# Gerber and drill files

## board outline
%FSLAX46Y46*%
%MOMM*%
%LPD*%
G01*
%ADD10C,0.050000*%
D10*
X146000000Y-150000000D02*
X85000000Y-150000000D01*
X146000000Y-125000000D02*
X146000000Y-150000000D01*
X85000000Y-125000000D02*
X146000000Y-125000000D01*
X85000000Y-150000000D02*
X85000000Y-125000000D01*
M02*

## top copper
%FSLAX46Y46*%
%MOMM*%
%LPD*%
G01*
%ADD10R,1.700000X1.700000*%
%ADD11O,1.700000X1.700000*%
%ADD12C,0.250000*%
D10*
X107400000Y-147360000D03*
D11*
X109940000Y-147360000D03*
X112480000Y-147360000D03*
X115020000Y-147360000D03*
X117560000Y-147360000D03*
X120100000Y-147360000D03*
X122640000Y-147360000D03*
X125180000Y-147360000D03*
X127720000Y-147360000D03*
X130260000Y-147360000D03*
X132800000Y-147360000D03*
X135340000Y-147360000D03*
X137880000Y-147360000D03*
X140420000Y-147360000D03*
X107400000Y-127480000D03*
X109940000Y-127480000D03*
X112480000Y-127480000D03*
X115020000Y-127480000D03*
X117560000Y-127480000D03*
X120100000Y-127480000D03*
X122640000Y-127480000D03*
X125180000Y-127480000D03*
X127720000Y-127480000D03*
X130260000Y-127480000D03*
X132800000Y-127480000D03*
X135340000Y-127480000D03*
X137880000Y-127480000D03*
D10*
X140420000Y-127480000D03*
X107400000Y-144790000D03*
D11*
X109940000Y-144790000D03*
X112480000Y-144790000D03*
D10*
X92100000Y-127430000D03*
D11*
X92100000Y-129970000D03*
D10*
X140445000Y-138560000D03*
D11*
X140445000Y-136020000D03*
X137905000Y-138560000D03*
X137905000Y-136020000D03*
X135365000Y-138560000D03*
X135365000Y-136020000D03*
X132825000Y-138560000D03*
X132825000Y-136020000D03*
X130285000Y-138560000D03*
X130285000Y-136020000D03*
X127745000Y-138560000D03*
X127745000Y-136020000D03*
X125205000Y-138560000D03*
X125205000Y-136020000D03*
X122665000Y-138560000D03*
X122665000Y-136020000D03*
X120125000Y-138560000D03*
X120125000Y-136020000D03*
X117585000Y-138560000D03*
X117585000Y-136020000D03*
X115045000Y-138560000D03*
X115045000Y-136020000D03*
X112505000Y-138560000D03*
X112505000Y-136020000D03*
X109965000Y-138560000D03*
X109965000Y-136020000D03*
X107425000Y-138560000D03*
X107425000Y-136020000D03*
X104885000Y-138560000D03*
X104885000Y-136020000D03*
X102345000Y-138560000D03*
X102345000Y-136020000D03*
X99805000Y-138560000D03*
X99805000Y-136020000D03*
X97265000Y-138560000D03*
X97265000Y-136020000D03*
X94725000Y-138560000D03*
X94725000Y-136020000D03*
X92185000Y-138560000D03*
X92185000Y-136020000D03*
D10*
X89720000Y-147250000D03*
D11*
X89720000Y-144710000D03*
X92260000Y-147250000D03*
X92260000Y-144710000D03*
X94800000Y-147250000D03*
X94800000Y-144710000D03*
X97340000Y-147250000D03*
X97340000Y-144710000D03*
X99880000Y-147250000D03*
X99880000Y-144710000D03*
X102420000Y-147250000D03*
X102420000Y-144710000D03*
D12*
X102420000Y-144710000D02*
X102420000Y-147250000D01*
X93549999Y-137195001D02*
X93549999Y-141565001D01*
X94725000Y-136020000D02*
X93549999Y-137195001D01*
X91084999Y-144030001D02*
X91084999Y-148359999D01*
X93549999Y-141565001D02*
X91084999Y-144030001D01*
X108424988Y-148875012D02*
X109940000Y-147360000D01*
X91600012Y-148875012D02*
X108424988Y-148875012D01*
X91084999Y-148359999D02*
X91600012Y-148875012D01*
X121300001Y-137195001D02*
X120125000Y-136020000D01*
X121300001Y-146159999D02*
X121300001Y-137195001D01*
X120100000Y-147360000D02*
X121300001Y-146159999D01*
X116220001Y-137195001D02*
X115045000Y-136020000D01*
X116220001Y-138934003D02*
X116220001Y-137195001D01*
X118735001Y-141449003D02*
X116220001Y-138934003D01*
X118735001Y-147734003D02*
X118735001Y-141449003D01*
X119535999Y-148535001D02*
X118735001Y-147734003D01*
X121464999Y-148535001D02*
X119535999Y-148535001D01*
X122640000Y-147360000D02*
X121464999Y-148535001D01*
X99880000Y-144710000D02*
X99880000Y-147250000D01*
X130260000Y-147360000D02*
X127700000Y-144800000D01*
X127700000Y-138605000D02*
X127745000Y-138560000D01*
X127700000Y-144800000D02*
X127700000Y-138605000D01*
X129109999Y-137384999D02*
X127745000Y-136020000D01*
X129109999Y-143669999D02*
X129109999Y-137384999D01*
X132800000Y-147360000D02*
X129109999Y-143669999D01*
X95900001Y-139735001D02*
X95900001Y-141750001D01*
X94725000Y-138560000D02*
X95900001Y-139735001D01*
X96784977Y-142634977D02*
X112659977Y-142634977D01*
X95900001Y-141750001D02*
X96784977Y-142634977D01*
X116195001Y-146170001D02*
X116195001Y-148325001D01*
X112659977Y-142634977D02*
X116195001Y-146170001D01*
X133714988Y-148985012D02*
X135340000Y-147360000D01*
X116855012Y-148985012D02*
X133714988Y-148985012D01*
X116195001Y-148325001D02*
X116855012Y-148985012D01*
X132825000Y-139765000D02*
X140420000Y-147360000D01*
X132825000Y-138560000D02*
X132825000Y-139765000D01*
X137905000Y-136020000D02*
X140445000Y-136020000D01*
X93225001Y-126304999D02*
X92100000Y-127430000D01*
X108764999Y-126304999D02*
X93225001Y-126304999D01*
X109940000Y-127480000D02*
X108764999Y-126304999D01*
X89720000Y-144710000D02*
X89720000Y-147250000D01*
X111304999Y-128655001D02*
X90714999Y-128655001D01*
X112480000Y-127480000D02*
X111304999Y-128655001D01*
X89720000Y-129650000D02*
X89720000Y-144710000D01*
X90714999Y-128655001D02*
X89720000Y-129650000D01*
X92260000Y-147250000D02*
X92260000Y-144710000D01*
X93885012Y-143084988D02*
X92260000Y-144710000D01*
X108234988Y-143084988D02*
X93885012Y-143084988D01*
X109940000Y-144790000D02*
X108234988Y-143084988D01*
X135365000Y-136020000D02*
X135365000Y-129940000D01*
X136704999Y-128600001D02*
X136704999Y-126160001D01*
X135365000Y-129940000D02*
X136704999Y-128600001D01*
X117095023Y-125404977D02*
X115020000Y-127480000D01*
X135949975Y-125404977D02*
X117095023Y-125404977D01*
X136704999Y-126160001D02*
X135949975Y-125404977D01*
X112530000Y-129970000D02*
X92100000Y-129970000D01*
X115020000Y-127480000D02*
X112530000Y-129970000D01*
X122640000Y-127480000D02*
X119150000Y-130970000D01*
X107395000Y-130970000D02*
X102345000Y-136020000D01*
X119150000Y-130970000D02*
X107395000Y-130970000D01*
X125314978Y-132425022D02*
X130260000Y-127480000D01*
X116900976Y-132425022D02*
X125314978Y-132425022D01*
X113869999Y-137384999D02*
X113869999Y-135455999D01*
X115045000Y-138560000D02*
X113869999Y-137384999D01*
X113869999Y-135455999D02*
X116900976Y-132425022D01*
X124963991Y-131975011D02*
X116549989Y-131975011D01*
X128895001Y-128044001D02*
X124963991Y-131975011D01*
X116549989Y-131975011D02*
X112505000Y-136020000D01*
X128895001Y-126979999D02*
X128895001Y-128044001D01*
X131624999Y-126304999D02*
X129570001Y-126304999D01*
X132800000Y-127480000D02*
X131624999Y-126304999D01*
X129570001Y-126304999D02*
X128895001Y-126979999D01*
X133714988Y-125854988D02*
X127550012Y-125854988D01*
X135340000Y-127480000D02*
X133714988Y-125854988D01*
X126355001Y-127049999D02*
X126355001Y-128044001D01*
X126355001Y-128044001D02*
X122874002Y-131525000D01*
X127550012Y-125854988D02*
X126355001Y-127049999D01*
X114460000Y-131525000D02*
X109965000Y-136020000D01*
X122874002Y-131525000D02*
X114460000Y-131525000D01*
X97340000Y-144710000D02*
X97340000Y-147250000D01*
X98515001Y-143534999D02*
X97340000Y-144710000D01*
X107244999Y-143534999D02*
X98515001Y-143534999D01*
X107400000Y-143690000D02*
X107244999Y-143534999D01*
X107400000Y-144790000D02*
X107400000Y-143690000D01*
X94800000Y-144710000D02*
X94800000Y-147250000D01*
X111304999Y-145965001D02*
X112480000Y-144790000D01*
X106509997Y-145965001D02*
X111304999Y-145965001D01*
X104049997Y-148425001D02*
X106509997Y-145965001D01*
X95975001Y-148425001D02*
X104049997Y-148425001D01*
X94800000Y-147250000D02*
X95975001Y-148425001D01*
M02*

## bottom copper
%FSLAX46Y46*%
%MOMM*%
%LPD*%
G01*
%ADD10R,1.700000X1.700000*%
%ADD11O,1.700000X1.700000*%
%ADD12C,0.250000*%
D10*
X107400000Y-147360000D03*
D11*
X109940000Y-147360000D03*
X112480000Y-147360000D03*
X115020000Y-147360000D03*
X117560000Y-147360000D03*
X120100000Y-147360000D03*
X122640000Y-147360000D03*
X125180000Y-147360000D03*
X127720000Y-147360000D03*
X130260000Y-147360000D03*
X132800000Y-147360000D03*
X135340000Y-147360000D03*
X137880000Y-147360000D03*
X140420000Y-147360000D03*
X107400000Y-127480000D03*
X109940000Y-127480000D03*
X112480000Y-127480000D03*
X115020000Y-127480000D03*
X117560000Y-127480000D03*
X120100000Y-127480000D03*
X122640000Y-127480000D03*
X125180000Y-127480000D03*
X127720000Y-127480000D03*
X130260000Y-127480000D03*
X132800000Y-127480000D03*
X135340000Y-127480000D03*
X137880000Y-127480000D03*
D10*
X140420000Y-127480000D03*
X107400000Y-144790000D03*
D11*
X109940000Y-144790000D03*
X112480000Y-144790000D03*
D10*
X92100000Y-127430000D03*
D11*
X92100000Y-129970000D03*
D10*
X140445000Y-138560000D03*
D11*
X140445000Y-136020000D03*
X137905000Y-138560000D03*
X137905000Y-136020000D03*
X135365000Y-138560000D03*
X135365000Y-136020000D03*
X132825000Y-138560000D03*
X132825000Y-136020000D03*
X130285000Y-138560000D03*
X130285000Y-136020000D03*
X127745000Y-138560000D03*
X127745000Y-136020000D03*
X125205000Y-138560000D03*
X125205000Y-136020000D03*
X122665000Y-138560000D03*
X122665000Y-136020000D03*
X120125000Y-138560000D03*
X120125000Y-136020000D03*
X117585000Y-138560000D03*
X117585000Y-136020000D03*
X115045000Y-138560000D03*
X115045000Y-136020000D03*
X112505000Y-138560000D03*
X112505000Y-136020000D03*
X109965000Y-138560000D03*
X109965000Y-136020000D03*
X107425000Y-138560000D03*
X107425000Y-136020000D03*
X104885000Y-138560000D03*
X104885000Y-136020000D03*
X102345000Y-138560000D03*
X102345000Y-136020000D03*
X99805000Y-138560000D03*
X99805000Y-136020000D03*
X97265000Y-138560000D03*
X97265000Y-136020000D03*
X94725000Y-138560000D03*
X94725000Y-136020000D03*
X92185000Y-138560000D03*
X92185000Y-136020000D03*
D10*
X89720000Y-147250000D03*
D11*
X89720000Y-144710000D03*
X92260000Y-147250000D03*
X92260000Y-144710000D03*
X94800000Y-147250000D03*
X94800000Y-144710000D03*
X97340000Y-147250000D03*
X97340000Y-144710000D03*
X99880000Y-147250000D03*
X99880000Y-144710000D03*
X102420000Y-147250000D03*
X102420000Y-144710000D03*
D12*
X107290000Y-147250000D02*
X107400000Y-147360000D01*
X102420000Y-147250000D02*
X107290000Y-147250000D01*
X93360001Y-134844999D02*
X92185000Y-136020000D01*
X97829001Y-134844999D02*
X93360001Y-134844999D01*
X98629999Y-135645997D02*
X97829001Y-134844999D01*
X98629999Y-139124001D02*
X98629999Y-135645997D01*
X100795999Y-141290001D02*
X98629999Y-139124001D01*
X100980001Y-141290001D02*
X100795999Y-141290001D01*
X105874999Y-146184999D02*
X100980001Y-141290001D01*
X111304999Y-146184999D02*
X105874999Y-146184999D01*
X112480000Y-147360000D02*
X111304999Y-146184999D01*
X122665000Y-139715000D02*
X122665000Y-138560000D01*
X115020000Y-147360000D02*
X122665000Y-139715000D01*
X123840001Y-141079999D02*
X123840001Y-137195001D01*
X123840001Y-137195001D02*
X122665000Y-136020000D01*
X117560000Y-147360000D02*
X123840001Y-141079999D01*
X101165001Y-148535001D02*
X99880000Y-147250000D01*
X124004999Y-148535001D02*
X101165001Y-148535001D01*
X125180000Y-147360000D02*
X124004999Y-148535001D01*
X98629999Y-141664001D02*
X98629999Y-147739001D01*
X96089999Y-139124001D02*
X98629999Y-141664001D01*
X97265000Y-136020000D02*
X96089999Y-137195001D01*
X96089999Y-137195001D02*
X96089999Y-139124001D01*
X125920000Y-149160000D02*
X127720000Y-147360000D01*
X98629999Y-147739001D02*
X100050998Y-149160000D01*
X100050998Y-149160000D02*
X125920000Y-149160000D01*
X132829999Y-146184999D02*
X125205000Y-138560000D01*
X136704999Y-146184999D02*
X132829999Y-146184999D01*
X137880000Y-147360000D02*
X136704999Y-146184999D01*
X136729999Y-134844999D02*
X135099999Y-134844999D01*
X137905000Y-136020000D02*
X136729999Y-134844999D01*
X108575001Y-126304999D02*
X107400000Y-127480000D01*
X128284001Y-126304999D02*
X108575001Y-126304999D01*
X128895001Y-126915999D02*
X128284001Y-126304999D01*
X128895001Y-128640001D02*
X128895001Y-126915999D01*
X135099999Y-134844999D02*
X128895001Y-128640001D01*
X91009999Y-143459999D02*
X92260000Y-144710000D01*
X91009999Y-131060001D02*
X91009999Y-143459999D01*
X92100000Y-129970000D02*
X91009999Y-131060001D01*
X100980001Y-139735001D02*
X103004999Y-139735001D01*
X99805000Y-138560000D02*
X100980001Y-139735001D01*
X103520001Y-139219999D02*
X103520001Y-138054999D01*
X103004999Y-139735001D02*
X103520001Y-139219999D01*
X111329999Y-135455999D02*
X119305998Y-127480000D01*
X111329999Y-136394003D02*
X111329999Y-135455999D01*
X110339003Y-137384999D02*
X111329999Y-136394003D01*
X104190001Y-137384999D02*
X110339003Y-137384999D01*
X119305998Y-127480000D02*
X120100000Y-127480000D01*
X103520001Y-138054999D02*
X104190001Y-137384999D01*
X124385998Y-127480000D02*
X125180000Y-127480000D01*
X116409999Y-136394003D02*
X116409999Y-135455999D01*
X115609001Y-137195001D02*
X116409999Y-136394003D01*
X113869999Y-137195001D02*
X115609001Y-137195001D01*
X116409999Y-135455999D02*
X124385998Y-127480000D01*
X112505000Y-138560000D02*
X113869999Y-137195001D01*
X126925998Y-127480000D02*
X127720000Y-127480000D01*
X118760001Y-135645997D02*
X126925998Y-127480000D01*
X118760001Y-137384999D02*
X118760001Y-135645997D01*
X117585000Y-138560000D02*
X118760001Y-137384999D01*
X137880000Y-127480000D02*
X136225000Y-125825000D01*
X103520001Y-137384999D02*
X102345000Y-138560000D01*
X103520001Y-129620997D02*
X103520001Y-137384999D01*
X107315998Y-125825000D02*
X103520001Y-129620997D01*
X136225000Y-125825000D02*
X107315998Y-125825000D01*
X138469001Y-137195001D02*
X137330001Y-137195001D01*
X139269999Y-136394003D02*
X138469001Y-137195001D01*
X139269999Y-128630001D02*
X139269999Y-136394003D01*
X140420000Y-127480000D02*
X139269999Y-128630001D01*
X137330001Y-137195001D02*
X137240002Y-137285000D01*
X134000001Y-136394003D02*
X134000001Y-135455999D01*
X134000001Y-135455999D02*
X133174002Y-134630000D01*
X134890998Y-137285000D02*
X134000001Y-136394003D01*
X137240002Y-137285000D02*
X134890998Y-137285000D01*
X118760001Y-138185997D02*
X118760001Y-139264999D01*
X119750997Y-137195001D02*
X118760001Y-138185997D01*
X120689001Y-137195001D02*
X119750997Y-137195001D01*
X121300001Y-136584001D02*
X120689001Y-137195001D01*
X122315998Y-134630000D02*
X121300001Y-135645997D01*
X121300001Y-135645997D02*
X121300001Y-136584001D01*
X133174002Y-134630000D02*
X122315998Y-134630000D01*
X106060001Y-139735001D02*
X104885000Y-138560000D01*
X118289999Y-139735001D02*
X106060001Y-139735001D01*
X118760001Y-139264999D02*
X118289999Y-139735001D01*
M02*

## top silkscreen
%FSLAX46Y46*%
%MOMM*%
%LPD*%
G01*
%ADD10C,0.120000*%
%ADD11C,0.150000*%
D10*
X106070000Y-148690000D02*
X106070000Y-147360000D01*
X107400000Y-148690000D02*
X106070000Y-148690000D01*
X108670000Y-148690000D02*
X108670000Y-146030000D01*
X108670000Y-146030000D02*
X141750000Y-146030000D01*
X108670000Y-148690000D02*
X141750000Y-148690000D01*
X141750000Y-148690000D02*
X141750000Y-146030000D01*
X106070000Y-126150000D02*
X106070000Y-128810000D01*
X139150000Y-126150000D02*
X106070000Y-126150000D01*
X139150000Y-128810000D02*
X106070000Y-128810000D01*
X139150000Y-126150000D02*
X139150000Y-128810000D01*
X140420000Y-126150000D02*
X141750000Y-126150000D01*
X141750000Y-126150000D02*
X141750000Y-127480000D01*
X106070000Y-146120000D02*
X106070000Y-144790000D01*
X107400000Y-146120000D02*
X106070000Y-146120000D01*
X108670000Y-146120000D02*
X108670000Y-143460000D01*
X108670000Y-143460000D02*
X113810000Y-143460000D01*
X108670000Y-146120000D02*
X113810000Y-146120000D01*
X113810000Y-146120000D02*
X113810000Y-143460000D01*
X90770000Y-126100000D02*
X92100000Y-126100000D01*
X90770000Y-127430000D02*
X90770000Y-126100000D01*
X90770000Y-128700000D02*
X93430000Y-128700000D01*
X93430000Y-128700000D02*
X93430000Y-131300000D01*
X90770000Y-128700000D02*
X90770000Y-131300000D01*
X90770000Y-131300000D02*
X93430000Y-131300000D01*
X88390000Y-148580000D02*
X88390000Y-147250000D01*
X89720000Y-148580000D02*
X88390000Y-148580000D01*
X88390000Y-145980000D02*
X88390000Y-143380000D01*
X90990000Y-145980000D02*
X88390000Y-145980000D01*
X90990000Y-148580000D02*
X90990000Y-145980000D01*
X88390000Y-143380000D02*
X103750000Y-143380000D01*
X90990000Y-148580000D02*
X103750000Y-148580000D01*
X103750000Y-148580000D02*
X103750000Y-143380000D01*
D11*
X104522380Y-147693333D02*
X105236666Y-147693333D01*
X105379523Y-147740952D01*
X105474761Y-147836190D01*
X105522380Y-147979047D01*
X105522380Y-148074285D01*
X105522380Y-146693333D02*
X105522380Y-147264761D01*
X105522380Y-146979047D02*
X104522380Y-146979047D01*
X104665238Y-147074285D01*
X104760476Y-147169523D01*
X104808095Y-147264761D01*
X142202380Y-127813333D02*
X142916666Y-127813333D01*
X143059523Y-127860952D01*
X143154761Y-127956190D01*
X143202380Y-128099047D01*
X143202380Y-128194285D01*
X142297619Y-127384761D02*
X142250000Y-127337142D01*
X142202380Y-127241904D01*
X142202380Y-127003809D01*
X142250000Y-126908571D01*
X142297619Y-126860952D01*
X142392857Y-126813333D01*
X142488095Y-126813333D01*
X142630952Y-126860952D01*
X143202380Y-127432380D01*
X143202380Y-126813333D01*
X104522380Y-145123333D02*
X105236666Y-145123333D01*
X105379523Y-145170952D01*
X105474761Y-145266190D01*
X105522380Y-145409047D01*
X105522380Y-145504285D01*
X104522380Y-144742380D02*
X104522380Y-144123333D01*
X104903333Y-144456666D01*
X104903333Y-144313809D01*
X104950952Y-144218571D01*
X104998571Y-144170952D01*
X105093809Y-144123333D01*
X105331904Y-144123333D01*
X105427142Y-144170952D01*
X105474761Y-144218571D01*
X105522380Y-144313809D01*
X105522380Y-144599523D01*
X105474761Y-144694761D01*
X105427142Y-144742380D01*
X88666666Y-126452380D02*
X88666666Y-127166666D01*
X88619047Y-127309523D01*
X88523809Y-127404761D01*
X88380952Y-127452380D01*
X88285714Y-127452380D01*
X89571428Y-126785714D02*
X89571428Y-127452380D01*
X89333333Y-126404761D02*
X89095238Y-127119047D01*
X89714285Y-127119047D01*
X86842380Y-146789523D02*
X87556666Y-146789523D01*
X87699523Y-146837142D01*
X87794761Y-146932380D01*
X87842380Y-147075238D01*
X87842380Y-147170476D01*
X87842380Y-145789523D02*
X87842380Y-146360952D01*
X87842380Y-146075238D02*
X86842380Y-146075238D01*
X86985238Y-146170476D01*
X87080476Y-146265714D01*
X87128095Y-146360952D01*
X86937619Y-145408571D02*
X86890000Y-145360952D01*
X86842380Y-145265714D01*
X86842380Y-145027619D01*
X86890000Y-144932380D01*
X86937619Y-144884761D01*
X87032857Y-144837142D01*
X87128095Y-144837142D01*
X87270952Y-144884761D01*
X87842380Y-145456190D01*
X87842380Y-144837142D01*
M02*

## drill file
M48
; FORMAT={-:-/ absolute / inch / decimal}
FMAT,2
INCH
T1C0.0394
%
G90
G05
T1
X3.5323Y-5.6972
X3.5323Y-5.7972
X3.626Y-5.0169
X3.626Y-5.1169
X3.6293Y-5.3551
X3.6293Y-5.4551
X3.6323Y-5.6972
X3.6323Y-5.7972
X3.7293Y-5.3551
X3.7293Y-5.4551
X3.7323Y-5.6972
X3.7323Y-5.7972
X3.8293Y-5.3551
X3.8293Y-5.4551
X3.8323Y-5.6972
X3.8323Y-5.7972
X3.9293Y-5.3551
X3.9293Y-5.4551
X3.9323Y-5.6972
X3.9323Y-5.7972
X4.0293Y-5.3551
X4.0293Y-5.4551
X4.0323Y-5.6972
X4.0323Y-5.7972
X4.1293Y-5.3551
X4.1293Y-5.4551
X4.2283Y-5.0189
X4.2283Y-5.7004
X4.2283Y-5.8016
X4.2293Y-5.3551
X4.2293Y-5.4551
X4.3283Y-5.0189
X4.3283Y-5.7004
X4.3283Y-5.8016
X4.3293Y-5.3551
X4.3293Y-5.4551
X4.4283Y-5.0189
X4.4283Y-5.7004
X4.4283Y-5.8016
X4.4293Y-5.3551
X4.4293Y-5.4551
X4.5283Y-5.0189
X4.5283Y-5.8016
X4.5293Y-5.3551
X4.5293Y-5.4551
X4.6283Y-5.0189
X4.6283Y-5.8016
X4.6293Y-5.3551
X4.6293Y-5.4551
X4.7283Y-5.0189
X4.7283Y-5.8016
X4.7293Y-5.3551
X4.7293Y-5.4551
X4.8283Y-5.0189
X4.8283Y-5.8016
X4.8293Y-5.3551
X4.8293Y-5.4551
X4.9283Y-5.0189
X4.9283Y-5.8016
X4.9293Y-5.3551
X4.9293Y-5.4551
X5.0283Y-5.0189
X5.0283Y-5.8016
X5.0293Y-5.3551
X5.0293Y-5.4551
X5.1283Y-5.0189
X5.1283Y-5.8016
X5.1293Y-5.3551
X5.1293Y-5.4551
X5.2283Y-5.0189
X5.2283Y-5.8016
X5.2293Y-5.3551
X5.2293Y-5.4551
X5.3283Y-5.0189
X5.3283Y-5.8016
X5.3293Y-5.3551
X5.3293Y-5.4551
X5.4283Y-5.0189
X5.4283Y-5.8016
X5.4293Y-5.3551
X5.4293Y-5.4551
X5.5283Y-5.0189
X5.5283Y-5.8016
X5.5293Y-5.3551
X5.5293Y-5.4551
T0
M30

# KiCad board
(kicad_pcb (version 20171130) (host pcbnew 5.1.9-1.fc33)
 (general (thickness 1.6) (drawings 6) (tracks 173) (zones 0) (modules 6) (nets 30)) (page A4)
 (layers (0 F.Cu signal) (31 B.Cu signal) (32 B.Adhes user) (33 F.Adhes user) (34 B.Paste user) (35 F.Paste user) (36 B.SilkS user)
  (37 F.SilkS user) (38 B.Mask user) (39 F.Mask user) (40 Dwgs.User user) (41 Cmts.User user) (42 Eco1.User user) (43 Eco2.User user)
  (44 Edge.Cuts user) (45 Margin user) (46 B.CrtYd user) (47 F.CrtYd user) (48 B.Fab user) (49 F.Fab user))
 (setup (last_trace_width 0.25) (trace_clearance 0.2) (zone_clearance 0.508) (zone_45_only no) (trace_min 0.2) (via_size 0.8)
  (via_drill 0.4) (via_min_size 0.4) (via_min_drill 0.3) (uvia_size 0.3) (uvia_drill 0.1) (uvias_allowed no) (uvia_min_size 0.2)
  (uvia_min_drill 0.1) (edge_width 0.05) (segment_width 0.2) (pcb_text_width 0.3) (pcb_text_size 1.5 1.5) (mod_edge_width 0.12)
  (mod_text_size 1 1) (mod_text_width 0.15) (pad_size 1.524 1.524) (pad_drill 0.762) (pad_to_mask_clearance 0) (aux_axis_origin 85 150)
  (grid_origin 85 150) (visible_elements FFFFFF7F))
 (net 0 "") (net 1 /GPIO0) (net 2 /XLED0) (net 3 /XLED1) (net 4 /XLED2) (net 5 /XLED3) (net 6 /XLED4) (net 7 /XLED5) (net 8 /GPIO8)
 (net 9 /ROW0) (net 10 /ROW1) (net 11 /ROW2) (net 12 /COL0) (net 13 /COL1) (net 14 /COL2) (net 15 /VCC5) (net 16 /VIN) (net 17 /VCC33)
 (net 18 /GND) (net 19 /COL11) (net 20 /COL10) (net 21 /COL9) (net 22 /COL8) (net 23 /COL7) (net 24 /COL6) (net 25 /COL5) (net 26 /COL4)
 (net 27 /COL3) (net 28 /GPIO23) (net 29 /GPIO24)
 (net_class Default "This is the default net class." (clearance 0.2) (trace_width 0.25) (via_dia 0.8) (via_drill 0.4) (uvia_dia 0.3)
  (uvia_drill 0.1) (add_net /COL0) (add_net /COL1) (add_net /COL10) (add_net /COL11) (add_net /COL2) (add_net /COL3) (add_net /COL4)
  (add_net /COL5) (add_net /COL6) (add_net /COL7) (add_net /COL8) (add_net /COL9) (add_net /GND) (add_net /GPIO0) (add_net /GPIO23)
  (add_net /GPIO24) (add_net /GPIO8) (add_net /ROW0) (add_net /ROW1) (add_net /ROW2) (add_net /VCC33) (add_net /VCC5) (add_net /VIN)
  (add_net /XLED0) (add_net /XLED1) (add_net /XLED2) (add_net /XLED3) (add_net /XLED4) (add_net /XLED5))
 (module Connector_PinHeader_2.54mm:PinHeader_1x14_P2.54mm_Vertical (layer F.Cu) (at 107.4 147.36 90)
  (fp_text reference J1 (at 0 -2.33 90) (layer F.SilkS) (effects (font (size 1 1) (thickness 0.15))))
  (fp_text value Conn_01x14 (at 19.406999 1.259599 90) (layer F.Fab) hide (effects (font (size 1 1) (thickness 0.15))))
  (fp_line (start -1.33 -1.33) (end 0 -1.33) (layer F.SilkS) (width 0.12))
  (fp_line (start -1.33 0) (end -1.33 -1.33) (layer F.SilkS) (width 0.12))
  (fp_line (start -1.33 1.27) (end 1.33 1.27) (layer F.SilkS) (width 0.12))
  (fp_line (start 1.33 1.27) (end 1.33 34.35) (layer F.SilkS) (width 0.12))
  (fp_line (start -1.33 1.27) (end -1.33 34.35) (layer F.SilkS) (width 0.12))
  (fp_line (start -1.33 34.35) (end 1.33 34.35) (layer F.SilkS) (width 0.12))
  (pad 1 thru_hole rect (at 0 0 90) (size 1.7 1.7) (drill 1) (layers *.Cu *.Mask) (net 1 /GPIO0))
  (pad 2 thru_hole oval (at 0 2.54 90) (size 1.7 1.7) (drill 1) (layers *.Cu *.Mask) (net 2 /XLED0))
  (pad 3 thru_hole oval (at 0 5.08 90) (size 1.7 1.7) (drill 1) (layers *.Cu *.Mask) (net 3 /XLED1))
  (pad 4 thru_hole oval (at 0 7.62 90) (size 1.7 1.7) (drill 1) (layers *.Cu *.Mask) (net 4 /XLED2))
  (pad 5 thru_hole oval (at 0 10.16 90) (size 1.7 1.7) (drill 1) (layers *.Cu *.Mask) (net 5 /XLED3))
  (pad 6 thru_hole oval (at 0 12.7 90) (size 1.7 1.7) (drill 1) (layers *.Cu *.Mask) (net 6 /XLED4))
  (pad 7 thru_hole oval (at 0 15.24 90) (size 1.7 1.7) (drill 1) (layers *.Cu *.Mask) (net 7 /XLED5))
  (pad 8 thru_hole oval (at 0 17.78 90) (size 1.7 1.7) (drill 1) (layers *.Cu *.Mask) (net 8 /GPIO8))
  (pad 9 thru_hole oval (at 0 20.32 90) (size 1.7 1.7) (drill 1) (layers *.Cu *.Mask) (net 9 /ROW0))
  (pad 10 thru_hole oval (at 0 22.86 90) (size 1.7 1.7) (drill 1) (layers *.Cu *.Mask) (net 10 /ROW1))
  (pad 11 thru_hole oval (at 0 25.4 90) (size 1.7 1.7) (drill 1) (layers *.Cu *.Mask) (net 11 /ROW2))
  (pad 12 thru_hole oval (at 0 27.94 90) (size 1.7 1.7) (drill 1) (layers *.Cu *.Mask) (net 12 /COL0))
  (pad 13 thru_hole oval (at 0 30.48 90) (size 1.7 1.7) (drill 1) (layers *.Cu *.Mask) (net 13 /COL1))
  (pad 14 thru_hole oval (at 0 33.02 90) (size 1.7 1.7) (drill 1) (layers *.Cu *.Mask) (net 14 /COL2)))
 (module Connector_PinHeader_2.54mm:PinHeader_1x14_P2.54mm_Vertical (layer F.Cu) (at 140.42 127.48 270)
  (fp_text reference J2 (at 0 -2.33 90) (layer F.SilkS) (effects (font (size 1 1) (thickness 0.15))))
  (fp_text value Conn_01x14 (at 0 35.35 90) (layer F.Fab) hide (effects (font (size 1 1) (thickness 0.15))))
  (fp_line (start -1.33 34.35) (end 1.33 34.35) (layer F.SilkS) (width 0.12))
  (fp_line (start -1.33 1.27) (end -1.33 34.35) (layer F.SilkS) (width 0.12))
  (fp_line (start 1.33 1.27) (end 1.33 34.35) (layer F.SilkS) (width 0.12))
  (fp_line (start -1.33 1.27) (end 1.33 1.27) (layer F.SilkS) (width 0.12))
  (fp_line (start -1.33 0) (end -1.33 -1.33) (layer F.SilkS) (width 0.12))
  (fp_line (start -1.33 -1.33) (end 0 -1.33) (layer F.SilkS) (width 0.12))
  (pad 14 thru_hole oval (at 0 33.02 270) (size 1.7 1.7) (drill 1) (layers *.Cu *.Mask) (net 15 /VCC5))
  (pad 13 thru_hole oval (at 0 30.48 270) (size 1.7 1.7) (drill 1) (layers *.Cu *.Mask) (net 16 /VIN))
  (pad 12 thru_hole oval (at 0 27.94 270) (size 1.7 1.7) (drill 1) (layers *.Cu *.Mask) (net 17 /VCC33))
  (pad 11 thru_hole oval (at 0 25.4 270) (size 1.7 1.7) (drill 1) (layers *.Cu *.Mask) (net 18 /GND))
  (pad 10 thru_hole oval (at 0 22.86 270) (size 1.7 1.7) (drill 1) (layers *.Cu *.Mask))
  (pad 9 thru_hole oval (at 0 20.32 270) (size 1.7 1.7) (drill 1) (layers *.Cu *.Mask) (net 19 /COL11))
  (pad 8 thru_hole oval (at 0 17.78 270) (size 1.7 1.7) (drill 1) (layers *.Cu *.Mask) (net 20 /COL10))
  (pad 7 thru_hole oval (at 0 15.24 270) (size 1.7 1.7) (drill 1) (layers *.Cu *.Mask) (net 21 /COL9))
  (pad 6 thru_hole oval (at 0 12.7 270) (size 1.7 1.7) (drill 1) (layers *.Cu *.Mask) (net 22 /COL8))
  (pad 5 thru_hole oval (at 0 10.16 270) (size 1.7 1.7) (drill 1) (layers *.Cu *.Mask) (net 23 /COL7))
  (pad 4 thru_hole oval (at 0 7.62 270) (size 1.7 1.7) (drill 1) (layers *.Cu *.Mask) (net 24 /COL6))
  (pad 3 thru_hole oval (at 0 5.08 270) (size 1.7 1.7) (drill 1) (layers *.Cu *.Mask) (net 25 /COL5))
  (pad 2 thru_hole oval (at 0 2.54 270) (size 1.7 1.7) (drill 1) (layers *.Cu *.Mask) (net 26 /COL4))
  (pad 1 thru_hole rect (at 0 0 270) (size 1.7 1.7) (drill 1) (layers *.Cu *.Mask) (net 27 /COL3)))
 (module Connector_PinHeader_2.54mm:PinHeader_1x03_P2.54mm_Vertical (layer F.Cu) (at 107.4 144.79 90)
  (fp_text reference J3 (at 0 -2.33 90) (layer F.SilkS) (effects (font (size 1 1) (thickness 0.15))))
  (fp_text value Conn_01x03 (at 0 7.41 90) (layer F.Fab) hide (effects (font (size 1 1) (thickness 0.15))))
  (fp_line (start -1.33 -1.33) (end 0 -1.33) (layer F.SilkS) (width 0.12))
  (fp_line (start -1.33 0) (end -1.33 -1.33) (layer F.SilkS) (width 0.12))
  (fp_line (start -1.33 1.27) (end 1.33 1.27) (layer F.SilkS) (width 0.12))
  (fp_line (start 1.33 1.27) (end 1.33 6.41) (layer F.SilkS) (width 0.12))
  (fp_line (start -1.33 1.27) (end -1.33 6.41) (layer F.SilkS) (width 0.12))
  (fp_line (start -1.33 6.41) (end 1.33 6.41) (layer F.SilkS) (width 0.12))
  (pad 1 thru_hole rect (at 0 0 90) (size 1.7 1.7) (drill 1) (layers *.Cu *.Mask) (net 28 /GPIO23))
  (pad 2 thru_hole oval (at 0 2.54 90) (size 1.7 1.7) (drill 1) (layers *.Cu *.Mask) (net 18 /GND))
  (pad 3 thru_hole oval (at 0 5.08 90) (size 1.7 1.7) (drill 1) (layers *.Cu *.Mask) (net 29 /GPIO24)))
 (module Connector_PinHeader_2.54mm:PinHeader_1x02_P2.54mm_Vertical (layer F.Cu) (at 92.1 127.43)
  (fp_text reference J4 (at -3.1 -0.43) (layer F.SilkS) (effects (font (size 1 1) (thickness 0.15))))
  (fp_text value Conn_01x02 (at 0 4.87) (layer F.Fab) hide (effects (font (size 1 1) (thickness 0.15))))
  (fp_line (start -1.33 -1.33) (end 0 -1.33) (layer F.SilkS) (width 0.12))
  (fp_line (start -1.33 0) (end -1.33 -1.33) (layer F.SilkS) (width 0.12))
  (fp_line (start -1.33 1.27) (end 1.33 1.27) (layer F.SilkS) (width 0.12))
  (fp_line (start 1.33 1.27) (end 1.33 3.87) (layer F.SilkS) (width 0.12))
  (fp_line (start -1.33 1.27) (end -1.33 3.87) (layer F.SilkS) (width 0.12))
  (fp_line (start -1.33 3.87) (end 1.33 3.87) (layer F.SilkS) (width 0.12))
  (pad 1 thru_hole rect (at 0 0) (size 1.7 1.7) (drill 1) (layers *.Cu *.Mask) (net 16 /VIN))
  (pad 2 thru_hole oval (at 0 2.54) (size 1.7 1.7) (drill 1) (layers *.Cu *.Mask) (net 18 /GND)))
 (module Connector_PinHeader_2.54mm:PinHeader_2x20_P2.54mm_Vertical (layer B.Cu) (at 140.445 138.56 90)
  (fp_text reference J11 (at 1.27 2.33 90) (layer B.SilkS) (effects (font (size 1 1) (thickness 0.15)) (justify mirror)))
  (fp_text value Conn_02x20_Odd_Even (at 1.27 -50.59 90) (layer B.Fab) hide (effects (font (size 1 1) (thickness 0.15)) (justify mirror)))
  (pad 1 thru_hole rect (at 0 0 90) (size 1.7 1.7) (drill 1) (layers *.Cu *.Mask))
  (pad 2 thru_hole oval (at 2.54 0 90) (size 1.7 1.7) (drill 1) (layers *.Cu *.Mask) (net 15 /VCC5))
  (pad 3 thru_hole oval (at 0 -2.54 90) (size 1.7 1.7) (drill 1) (layers *.Cu *.Mask))
  (pad 4 thru_hole oval (at 2.54 -2.54 90) (size 1.7 1.7) (drill 1) (layers *.Cu *.Mask) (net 15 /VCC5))
  (pad 5 thru_hole oval (at 0 -5.08 90) (size 1.7 1.7) (drill 1) (layers *.Cu *.Mask))
  (pad 6 thru_hole oval (at 2.54 -5.08 90) (size 1.7 1.7) (drill 1) (layers *.Cu *.Mask) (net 18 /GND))
  (pad 7 thru_hole oval (at 0 -7.62 90) (size 1.7 1.7) (drill 1) (layers *.Cu *.Mask) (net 14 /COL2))
  (pad 8 thru_hole oval (at 2.54 -7.62 90) (size 1.7 1.7) (drill 1) (layers *.Cu *.Mask))
  (pad 9 thru_hole oval (at 0 -10.16 90) (size 1.7 1.7) (drill 1) (layers *.Cu *.Mask))
  (pad 10 thru_hole oval (at 2.54 -10.16 90) (size 1.7 1.7) (drill 1) (layers *.Cu *.Mask))
  (pad 11 thru_hole oval (at 0 -12.7 90) (size 1.7 1.7) (drill 1) (layers *.Cu *.Mask) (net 10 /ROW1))
  (pad 12 thru_hole oval (at 2.54 -12.7 90) (size 1.7 1.7) (drill 1) (layers *.Cu *.Mask) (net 11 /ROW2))
  (pad 13 thru_hole oval (at 0 -15.24 90) (size 1.7 1.7) (drill 1) (layers *.Cu *.Mask) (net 13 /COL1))
  (pad 14 thru_hole oval (at 2.54 -15.24 90) (size 1.7 1.7) (drill 1) (layers *.Cu *.Mask))
  (pad 15 thru_hole oval (at 0 -17.78 90) (size 1.7 1.7) (drill 1) (layers *.Cu *.Mask) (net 4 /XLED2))
  (pad 16 thru_hole oval (at 2.54 -17.78 90) (size 1.7 1.7) (drill 1) (layers *.Cu *.Mask) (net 5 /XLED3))
  (pad 17 thru_hole oval (at 0 -20.32 90) (size 1.7 1.7) (drill 1) (layers *.Cu *.Mask))
  (pad 18 thru_hole oval (at 2.54 -20.32 90) (size 1.7 1.7) (drill 1) (layers *.Cu *.Mask) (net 6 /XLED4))
  (pad 19 thru_hole oval (at 0 -22.86 90) (size 1.7 1.7) (drill 1) (layers *.Cu *.Mask) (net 22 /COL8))
  (pad 20 thru_hole oval (at 2.54 -22.86 90) (size 1.7 1.7) (drill 1) (layers *.Cu *.Mask))
  (pad 21 thru_hole oval (at 0 -25.4 90) (size 1.7 1.7) (drill 1) (layers *.Cu *.Mask) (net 23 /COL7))
  (pad 22 thru_hole oval (at 2.54 -25.4 90) (size 1.7 1.7) (drill 1) (layers *.Cu *.Mask) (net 7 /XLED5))
  (pad 23 thru_hole oval (at 0 -27.94 90) (size 1.7 1.7) (drill 1) (layers *.Cu *.Mask) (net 21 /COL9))
  (pad 24 thru_hole oval (at 2.54 -27.94 90) (size 1.7 1.7) (drill 1) (layers *.Cu *.Mask) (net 24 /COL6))
  (pad 25 thru_hole oval (at 0 -30.48 90) (size 1.7 1.7) (drill 1) (layers *.Cu *.Mask))
  (pad 26 thru_hole oval (at 2.54 -30.48 90) (size 1.7 1.7) (drill 1) (layers *.Cu *.Mask) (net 25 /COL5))
  (pad 27 thru_hole oval (at 0 -33.02 90) (size 1.7 1.7) (drill 1) (layers *.Cu *.Mask))
  (pad 28 thru_hole oval (at 2.54 -33.02 90) (size 1.7 1.7) (drill 1) (layers *.Cu *.Mask))
  (pad 29 thru_hole oval (at 0 -35.56 90) (size 1.7 1.7) (drill 1) (layers *.Cu *.Mask) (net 27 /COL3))
  (pad 30 thru_hole oval (at 2.54 -35.56 90) (size 1.7 1.7) (drill 1) (layers *.Cu *.Mask))
  (pad 31 thru_hole oval (at 0 -38.1 90) (size 1.7 1.7) (drill 1) (layers *.Cu *.Mask) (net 26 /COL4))
  (pad 32 thru_hole oval (at 2.54 -38.1 90) (size 1.7 1.7) (drill 1) (layers *.Cu *.Mask) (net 20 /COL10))
  (pad 33 thru_hole oval (at 0 -40.64 90) (size 1.7 1.7) (drill 1) (layers *.Cu *.Mask) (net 19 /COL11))
  (pad 34 thru_hole oval (at 2.54 -40.64 90) (size 1.7 1.7) (drill 1) (layers *.Cu *.Mask))
  (pad 35 thru_hole oval (at 0 -43.18 90) (size 1.7 1.7) (drill 1) (layers *.Cu *.Mask))
  (pad 36 thru_hole oval (at 2.54 -43.18 90) (size 1.7 1.7) (drill 1) (layers *.Cu *.Mask) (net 9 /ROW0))
  (pad 37 thru_hole oval (at 0 -45.72 90) (size 1.7 1.7) (drill 1) (layers *.Cu *.Mask) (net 12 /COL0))
  (pad 38 thru_hole oval (at 2.54 -45.72 90) (size 1.7 1.7) (drill 1) (layers *.Cu *.Mask) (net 2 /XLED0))
  (pad 39 thru_hole oval (at 0 -48.26 90) (size 1.7 1.7) (drill 1) (layers *.Cu *.Mask))
  (pad 40 thru_hole oval (at 2.54 -48.26 90) (size 1.7 1.7) (drill 1) (layers *.Cu *.Mask) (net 3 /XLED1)))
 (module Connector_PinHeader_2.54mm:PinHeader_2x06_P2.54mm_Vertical (layer F.Cu) (at 89.72 147.25 90)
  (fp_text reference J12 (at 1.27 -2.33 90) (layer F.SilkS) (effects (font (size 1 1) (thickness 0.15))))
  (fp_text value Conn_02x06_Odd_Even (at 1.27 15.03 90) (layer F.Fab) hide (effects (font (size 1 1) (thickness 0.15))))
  (fp_line (start -1.33 -1.33) (end 0 -1.33) (layer F.SilkS) (width 0.12))
  (fp_line (start -1.33 0) (end -1.33 -1.33) (layer F.SilkS) (width 0.12))
  (fp_line (start 1.27 -1.33) (end 3.87 -1.33) (layer F.SilkS) (width 0.12))
  (fp_line (start 1.27 1.27) (end 1.27 -1.33) (layer F.SilkS) (width 0.12))
  (fp_line (start -1.33 1.27) (end 1.27 1.27) (layer F.SilkS) (width 0.12))
  (fp_line (start 3.87 -1.33) (end 3.87 14.03) (layer F.SilkS) (width 0.12))
  (fp_line (start -1.33 1.27) (end -1.33 14.03) (layer F.SilkS) (width 0.12))
  (fp_line (start -1.33 14.03) (end 3.87 14.03) (layer F.SilkS) (width 0.12))
  (pad 1 thru_hole rect (at 0 0 90) (size 1.7 1.7) (drill 1) (layers *.Cu *.Mask) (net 17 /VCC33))
  (pad 2 thru_hole oval (at 2.54 0 90) (size 1.7 1.7) (drill 1) (layers *.Cu *.Mask) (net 17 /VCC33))
  (pad 3 thru_hole oval (at 0 2.54 90) (size 1.7 1.7) (drill 1) (layers *.Cu *.Mask) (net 18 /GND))
  (pad 4 thru_hole oval (at 2.54 2.54 90) (size 1.7 1.7) (drill 1) (layers *.Cu *.Mask) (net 18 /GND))
  (pad 5 thru_hole oval (at 0 5.08 90) (size 1.7 1.7) (drill 1) (layers *.Cu *.Mask) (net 29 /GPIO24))
  (pad 6 thru_hole oval (at 2.54 5.08 90) (size 1.7 1.7) (drill 1) (layers *.Cu *.Mask) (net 29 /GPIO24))
  (pad 7 thru_hole oval (at 0 7.62 90) (size 1.7 1.7) (drill 1) (layers *.Cu *.Mask) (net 28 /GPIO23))
  (pad 8 thru_hole oval (at 2.54 7.62 90) (size 1.7 1.7) (drill 1) (layers *.Cu *.Mask) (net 28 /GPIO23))
  (pad 9 thru_hole oval (at 0 10.16 90) (size 1.7 1.7) (drill 1) (layers *.Cu *.Mask) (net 8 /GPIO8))
  (pad 10 thru_hole oval (at 2.54 10.16 90) (size 1.7 1.7) (drill 1) (layers *.Cu *.Mask) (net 8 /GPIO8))
  (pad 11 thru_hole oval (at 0 12.7 90) (size 1.7 1.7) (drill 1) (layers *.Cu *.Mask) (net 1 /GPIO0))
  (pad 12 thru_hole oval (at 2.54 12.7 90) (size 1.7 1.7) (drill 1) (layers *.Cu *.Mask) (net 1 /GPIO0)))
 (gr_line (start 146 150) (end 85 150) (layer Edge.Cuts) (width 0.05))
 (gr_line (start 146 125) (end 146 150) (layer Edge.Cuts) (width 0.05))
 (gr_line (start 85 125) (end 146 125) (layer Edge.Cuts) (width 0.05))
 (gr_line (start 85 150) (end 85 125) (layer Edge.Cuts) (width 0.05))
 (segment (start 102.42 144.71) (end 102.42 147.25) (width 0.25) (layer F.Cu) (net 1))
 (segment (start 107.29 147.25) (end 107.4 147.36) (width 0.25) (layer B.Cu) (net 1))
 (segment (start 102.42 147.25) (end 107.29 147.25) (width 0.25) (layer B.Cu) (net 1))
 (segment (start 93.549999 137.195001) (end 93.549999 141.565001) (width 0.25) (layer F.Cu) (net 2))
 (segment (start 94.725 136.02) (end 93.549999 137.195001) (width 0.25) (layer F.Cu) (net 2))
 (segment (start 91.084999 144.030001) (end 91.084999 148.359999) (width 0.25) (layer F.Cu) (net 2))
 (segment (start 93.549999 141.565001) (end 91.084999 144.030001) (width 0.25) (layer F.Cu) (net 2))
 (segment (start 108.424988 148.875012) (end 109.94 147.36) (width 0.25) (layer F.Cu) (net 2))
 (segment (start 91.600012 148.875012) (end 108.424988 148.875012) (width 0.25) (layer F.Cu) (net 2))
 (segment (start 91.084999 148.359999) (end 91.600012 148.875012) (width 0.25) (layer F.Cu) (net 2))
 (segment (start 93.360001 134.844999) (end 92.185 136.02) (width 0.25) (layer B.Cu) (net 3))
 (segment (start 97.829001 134.844999) (end 93.360001 134.844999) (width 0.25) (layer B.Cu) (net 3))
 (segment (start 98.629999 135.645997) (end 97.829001 134.844999) (width 0.25) (layer B.Cu) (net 3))
 (segment (start 98.629999 139.124001) (end 98.629999 135.645997) (width 0.25) (layer B.Cu) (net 3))
 (segment (start 100.795999 141.290001) (end 98.629999 139.124001) (width 0.25) (layer B.Cu) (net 3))
 (segment (start 100.980001 141.290001) (end 100.795999 141.290001) (width 0.25) (layer B.Cu) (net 3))
 (segment (start 105.874999 146.184999) (end 100.980001 141.290001) (width 0.25) (layer B.Cu) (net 3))
 (segment (start 111.304999 146.184999) (end 105.874999 146.184999) (width 0.25) (layer B.Cu) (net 3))
 (segment (start 112.48 147.36) (end 111.304999 146.184999) (width 0.25) (layer B.Cu) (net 3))
 (segment (start 122.665 139.715) (end 122.665 138.56) (width 0.25) (layer B.Cu) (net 4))
 (segment (start 115.02 147.36) (end 122.665 139.715) (width 0.25) (layer B.Cu) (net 4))
 (segment (start 123.840001 141.079999) (end 123.840001 137.195001) (width 0.25) (layer B.Cu) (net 5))
 (segment (start 123.840001 137.195001) (end 122.665 136.02) (width 0.25) (layer B.Cu) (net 5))
 (segment (start 117.56 147.36) (end 123.840001 141.079999) (width 0.25) (layer B.Cu) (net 5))
 (segment (start 121.300001 137.195001) (end 120.125 136.02) (width 0.25) (layer F.Cu) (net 6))
 (segment (start 121.300001 146.159999) (end 121.300001 137.195001) (width 0.25) (layer F.Cu) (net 6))
 (segment (start 120.1 147.36) (end 121.300001 146.159999) (width 0.25) (layer F.Cu) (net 6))
 (segment (start 116.220001 137.195001) (end 115.045 136.02) (width 0.25) (layer F.Cu) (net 7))
 (segment (start 116.220001 138.934003) (end 116.220001 137.195001) (width 0.25) (layer F.Cu) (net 7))
 (segment (start 118.735001 141.449003) (end 116.220001 138.934003) (width 0.25) (layer F.Cu) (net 7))
 (segment (start 118.735001 147.734003) (end 118.735001 141.449003) (width 0.25) (layer F.Cu) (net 7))
 (segment (start 119.535999 148.535001) (end 118.735001 147.734003) (width 0.25) (layer F.Cu) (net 7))
 (segment (start 121.464999 148.535001) (end 119.535999 148.535001) (width 0.25) (layer F.Cu) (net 7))
 (segment (start 122.64 147.36) (end 121.464999 148.535001) (width 0.25) (layer F.Cu) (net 7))
 (segment (start 99.88 144.71) (end 99.88 147.25) (width 0.25) (layer F.Cu) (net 8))
 (segment (start 101.165001 148.535001) (end 99.88 147.25) (width 0.25) (layer B.Cu) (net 8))
 (segment (start 124.004999 148.535001) (end 101.165001 148.535001) (width 0.25) (layer B.Cu) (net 8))
 (segment (start 125.18 147.36) (end 124.004999 148.535001) (width 0.25) (layer B.Cu) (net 8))
 (segment (start 98.629999 141.664001) (end 98.629999 147.739001) (width 0.25) (layer B.Cu) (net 9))
 (segment (start 96.089999 139.124001) (end 98.629999 141.664001) (width 0.25) (layer B.Cu) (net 9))
 (segment (start 97.265 136.02) (end 96.089999 137.195001) (width 0.25) (layer B.Cu) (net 9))
 (segment (start 96.089999 137.195001) (end 96.089999 139.124001) (width 0.25) (layer B.Cu) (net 9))
 (segment (start 125.92 149.16) (end 127.72 147.36) (width 0.25) (layer B.Cu) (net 9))
 (segment (start 98.629999 147.739001) (end 100.050998 149.16) (width 0.25) (layer B.Cu) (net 9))
 (segment (start 100.050998 149.16) (end 125.92 149.16) (width 0.25) (layer B.Cu) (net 9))
 (segment (start 130.26 147.36) (end 127.7 144.8) (width 0.25) (layer F.Cu) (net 10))
 (segment (start 127.7 138.605) (end 127.745 138.56) (width 0.25) (layer F.Cu) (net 10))
 (segment (start 127.7 144.8) (end 127.7 138.605) (width 0.25) (layer F.Cu) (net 10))
 (segment (start 129.109999 137.384999) (end 127.745 136.02) (width 0.25) (layer F.Cu) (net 11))
 (segment (start 129.109999 143.669999) (end 129.109999 137.384999) (width 0.25) (layer F.Cu) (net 11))
 (segment (start 132.8 147.36) (end 129.109999 143.669999) (width 0.25) (layer F.Cu) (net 11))
 (segment (start 95.900001 139.735001) (end 95.900001 141.750001) (width 0.25) (layer F.Cu) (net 12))
 (segment (start 94.725 138.56) (end 95.900001 139.735001) (width 0.25) (layer F.Cu) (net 12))
 (segment (start 96.784977 142.634977) (end 112.659977 142.634977) (width 0.25) (layer F.Cu) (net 12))
 (segment (start 95.900001 141.750001) (end 96.784977 142.634977) (width 0.25) (layer F.Cu) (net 12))
 (segment (start 116.195001 146.170001) (end 116.195001 148.325001) (width 0.25) (layer F.Cu) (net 12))
 (segment (start 112.659977 142.634977) (end 116.195001 146.170001) (width 0.25) (layer F.Cu) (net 12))
 (segment (start 133.714988 148.985012) (end 135.34 147.36) (width 0.25) (layer F.Cu) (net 12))
 (segment (start 116.855012 148.985012) (end 133.714988 148.985012) (width 0.25) (layer F.Cu) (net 12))
 (segment (start 116.195001 148.325001) (end 116.855012 148.985012) (width 0.25) (layer F.Cu) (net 12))
 (segment (start 132.829999 146.184999) (end 125.205 138.56) (width 0.25) (layer B.Cu) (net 13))
 (segment (start 136.704999 146.184999) (end 132.829999 146.184999) (width 0.25) (layer B.Cu) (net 13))
 (segment (start 137.88 147.36) (end 136.704999 146.184999) (width 0.25) (layer B.Cu) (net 13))
 (segment (start 132.825 139.765) (end 140.42 147.36) (width 0.25) (layer F.Cu) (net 14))
 (segment (start 132.825 138.56) (end 132.825 139.765) (width 0.25) (layer F.Cu) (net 14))
 (segment (start 137.905 136.02) (end 140.445 136.02) (width 0.25) (layer F.Cu) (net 15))
 (segment (start 136.729999 134.844999) (end 135.099999 134.844999) (width 0.25) (layer B.Cu) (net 15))
 (segment (start 137.905 136.02) (end 136.729999 134.844999) (width 0.25) (layer B.Cu) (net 15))
 (segment (start 108.575001 126.304999) (end 107.4 127.48) (width 0.25) (layer B.Cu) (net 15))
 (segment (start 128.284001 126.304999) (end 108.575001 126.304999) (width 0.25) (layer B.Cu) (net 15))
 (segment (start 128.895001 126.915999) (end 128.284001 126.304999) (width 0.25) (layer B.Cu) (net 15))
 (segment (start 128.895001 128.640001) (end 128.895001 126.915999) (width 0.25) (layer B.Cu) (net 15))
 (segment (start 135.099999 134.844999) (end 128.895001 128.640001) (width 0.25) (layer B.Cu) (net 15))
 (segment (start 93.225001 126.304999) (end 92.1 127.43) (width 0.25) (layer F.Cu) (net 16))
 (segment (start 108.764999 126.304999) (end 93.225001 126.304999) (width 0.25) (layer F.Cu) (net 16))
 (segment (start 109.94 127.48) (end 108.764999 126.304999) (width 0.25) (layer F.Cu) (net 16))
 (segment (start 89.72 144.71) (end 89.72 147.25) (width 0.25) (layer F.Cu) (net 17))
 (segment (start 111.304999 128.655001) (end 90.714999 128.655001) (width 0.25) (layer F.Cu) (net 17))
 (segment (start 112.48 127.48) (end 111.304999 128.655001) (width 0.25) (layer F.Cu) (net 17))
 (segment (start 89.72 129.65) (end 89.72 144.71) (width 0.25) (layer F.Cu) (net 17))
 (segment (start 90.714999 128.655001) (end 89.72 129.65) (width 0.25) (layer F.Cu) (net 17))
 (segment (start 92.26 147.25) (end 92.26 144.71) (width 0.25) (layer F.Cu) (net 18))
 (segment (start 93.885012 143.084988) (end 92.26 144.71) (width 0.25) (layer F.Cu) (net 18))
 (segment (start 108.234988 143.084988) (end 93.885012 143.084988) (width 0.25) (layer F.Cu) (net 18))
 (segment (start 109.94 144.79) (end 108.234988 143.084988) (width 0.25) (layer F.Cu) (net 18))
 (segment (start 135.365 136.02) (end 135.365 129.94) (width 0.25) (layer F.Cu) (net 18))
 (segment (start 136.704999 128.600001) (end 136.704999 126.160001) (width 0.25) (layer F.Cu) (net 18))
 (segment (start 135.365 129.94) (end 136.704999 128.600001) (width 0.25) (layer F.Cu) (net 18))
 (segment (start 117.095023 125.404977) (end 115.02 127.48) (width 0.25) (layer F.Cu) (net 18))
 (segment (start 135.949975 125.404977) (end 117.095023 125.404977) (width 0.25) (layer F.Cu) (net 18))
 (segment (start 136.704999 126.160001) (end 135.949975 125.404977) (width 0.25) (layer F.Cu) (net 18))
 (segment (start 112.53 129.97) (end 92.1 129.97) (width 0.25) (layer F.Cu) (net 18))
 (segment (start 115.02 127.48) (end 112.53 129.97) (width 0.25) (layer F.Cu) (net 18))
 (segment (start 91.009999 143.459999) (end 92.26 144.71) (width 0.25) (layer B.Cu) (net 18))
 (segment (start 91.009999 131.060001) (end 91.009999 143.459999) (width 0.25) (layer B.Cu) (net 18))
 (segment (start 92.1 129.97) (end 91.009999 131.060001) (width 0.25) (layer B.Cu) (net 18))
 (segment (start 100.980001 139.735001) (end 103.004999 139.735001) (width 0.25) (layer B.Cu) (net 19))
 (segment (start 99.805 138.56) (end 100.980001 139.735001) (width 0.25) (layer B.Cu) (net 19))
 (segment (start 103.520001 139.219999) (end 103.520001 138.054999) (width 0.25) (layer B.Cu) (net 19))
 (segment (start 103.004999 139.735001) (end 103.520001 139.219999) (width 0.25) (layer B.Cu) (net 19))
 (segment (start 111.329999 135.455999) (end 119.305998 127.48) (width 0.25) (layer B.Cu) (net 19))
 (segment (start 111.329999 136.394003) (end 111.329999 135.455999) (width 0.25) (layer B.Cu) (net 19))
 (segment (start 110.339003 137.384999) (end 111.329999 136.394003) (width 0.25) (layer B.Cu) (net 19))
 (segment (start 104.190001 137.384999) (end 110.339003 137.384999) (width 0.25) (layer B.Cu) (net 19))
 (segment (start 119.305998 127.48) (end 120.1 127.48) (width 0.25) (layer B.Cu) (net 19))
 (segment (start 103.520001 138.054999) (end 104.190001 137.384999) (width 0.25) (layer B.Cu) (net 19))
 (segment (start 122.64 127.48) (end 119.15 130.97) (width 0.25) (layer F.Cu) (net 20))
 (segment (start 107.395 130.97) (end 102.345 136.02) (width 0.25) (layer F.Cu) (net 20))
 (segment (start 119.15 130.97) (end 107.395 130.97) (width 0.25) (layer F.Cu) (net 20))
 (segment (start 124.385998 127.48) (end 125.18 127.48) (width 0.25) (layer B.Cu) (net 21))
 (segment (start 116.409999 136.394003) (end 116.409999 135.455999) (width 0.25) (layer B.Cu) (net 21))
 (segment (start 115.609001 137.195001) (end 116.409999 136.394003) (width 0.25) (layer B.Cu) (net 21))
 (segment (start 113.869999 137.195001) (end 115.609001 137.195001) (width 0.25) (layer B.Cu) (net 21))
 (segment (start 116.409999 135.455999) (end 124.385998 127.48) (width 0.25) (layer B.Cu) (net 21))
 (segment (start 112.505 138.56) (end 113.869999 137.195001) (width 0.25) (layer B.Cu) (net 21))
 (segment (start 126.925998 127.48) (end 127.72 127.48) (width 0.25) (layer B.Cu) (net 22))
 (segment (start 118.760001 135.645997) (end 126.925998 127.48) (width 0.25) (layer B.Cu) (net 22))
 (segment (start 118.760001 137.384999) (end 118.760001 135.645997) (width 0.25) (layer B.Cu) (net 22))
 (segment (start 117.585 138.56) (end 118.760001 137.384999) (width 0.25) (layer B.Cu) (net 22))
 (segment (start 125.314978 132.425022) (end 130.26 127.48) (width 0.25) (layer F.Cu) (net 23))
 (segment (start 116.900976 132.425022) (end 125.314978 132.425022) (width 0.25) (layer F.Cu) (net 23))
 (segment (start 113.869999 137.384999) (end 113.869999 135.455999) (width 0.25) (layer F.Cu) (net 23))
 (segment (start 115.045 138.56) (end 113.869999 137.384999) (width 0.25) (layer F.Cu) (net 23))
 (segment (start 113.869999 135.455999) (end 116.900976 132.425022) (width 0.25) (layer F.Cu) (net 23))
 (segment (start 124.963991 131.975011) (end 116.549989 131.975011) (width 0.25) (layer F.Cu) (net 24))
 (segment (start 128.895001 128.044001) (end 124.963991 131.975011) (width 0.25) (layer F.Cu) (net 24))
 (segment (start 116.549989 131.975011) (end 112.505 136.02) (width 0.25) (layer F.Cu) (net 24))
 (segment (start 128.895001 126.979999) (end 128.895001 128.044001) (width 0.25) (layer F.Cu) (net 24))
 (segment (start 131.624999 126.304999) (end 129.570001 126.304999) (width 0.25) (layer F.Cu) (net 24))
 (segment (start 132.8 127.48) (end 131.624999 126.304999) (width 0.25) (layer F.Cu) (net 24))
 (segment (start 129.570001 126.304999) (end 128.895001 126.979999) (width 0.25) (layer F.Cu) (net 24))
 (segment (start 133.714988 125.854988) (end 127.550012 125.854988) (width 0.25) (layer F.Cu) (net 25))
 (segment (start 135.34 127.48) (end 133.714988 125.854988) (width 0.25) (layer F.Cu) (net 25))
 (segment (start 126.355001 127.049999) (end 126.355001 128.044001) (width 0.25) (layer F.Cu) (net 25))
 (segment (start 126.355001 128.044001) (end 122.874002 131.525) (width 0.25) (layer F.Cu) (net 25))
 (segment (start 127.550012 125.854988) (end 126.355001 127.049999) (width 0.25) (layer F.Cu) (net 25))
 (segment (start 114.46 131.525) (end 109.965 136.02) (width 0.25) (layer F.Cu) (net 25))
 (segment (start 122.874002 131.525) (end 114.46 131.525) (width 0.25) (layer F.Cu) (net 25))
 (segment (start 137.88 127.48) (end 136.225 125.825) (width 0.25) (layer B.Cu) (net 26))
 (segment (start 103.520001 137.384999) (end 102.345 138.56) (width 0.25) (layer B.Cu) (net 26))
 (segment (start 103.520001 129.620997) (end 103.520001 137.384999) (width 0.25) (layer B.Cu) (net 26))
 (segment (start 107.315998 125.825) (end 103.520001 129.620997) (width 0.25) (layer B.Cu) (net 26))
 (segment (start 136.225 125.825) (end 107.315998 125.825) (width 0.25) (layer B.Cu) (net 26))
 (segment (start 138.469001 137.195001) (end 137.330001 137.195001) (width 0.25) (layer B.Cu) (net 27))
 (segment (start 139.269999 136.394003) (end 138.469001 137.195001) (width 0.25) (layer B.Cu) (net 27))
 (segment (start 139.269999 128.630001) (end 139.269999 136.394003) (width 0.25) (layer B.Cu) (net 27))
 (segment (start 140.42 127.48) (end 139.269999 128.630001) (width 0.25) (layer B.Cu) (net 27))
 (segment (start 137.330001 137.195001) (end 137.240002 137.285) (width 0.25) (layer B.Cu) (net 27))
 (segment (start 134.000001 136.394003) (end 134.000001 135.455999) (width 0.25) (layer B.Cu) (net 27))
 (segment (start 134.000001 135.455999) (end 133.174002 134.63) (width 0.25) (layer B.Cu) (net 27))
 (segment (start 134.890998 137.285) (end 134.000001 136.394003) (width 0.25) (layer B.Cu) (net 27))
 (segment (start 137.240002 137.285) (end 134.890998 137.285) (width 0.25) (layer B.Cu) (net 27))
 (segment (start 118.760001 138.185997) (end 118.760001 139.264999) (width 0.25) (layer B.Cu) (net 27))
 (segment (start 119.750997 137.195001) (end 118.760001 138.185997) (width 0.25) (layer B.Cu) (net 27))
 (segment (start 120.689001 137.195001) (end 119.750997 137.195001) (width 0.25) (layer B.Cu) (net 27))
 (segment (start 121.300001 136.584001) (end 120.689001 137.195001) (width 0.25) (layer B.Cu) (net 27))
 (segment (start 122.315998 134.63) (end 121.300001 135.645997) (width 0.25) (layer B.Cu) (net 27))
 (segment (start 121.300001 135.645997) (end 121.300001 136.584001) (width 0.25) (layer B.Cu) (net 27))
 (segment (start 133.174002 134.63) (end 122.315998 134.63) (width 0.25) (layer B.Cu) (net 27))
 (segment (start 106.060001 139.735001) (end 104.885 138.56) (width 0.25) (layer B.Cu) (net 27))
 (segment (start 118.289999 139.735001) (end 106.060001 139.735001) (width 0.25) (layer B.Cu) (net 27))
 (segment (start 118.760001 139.264999) (end 118.289999 139.735001) (width 0.25) (layer B.Cu) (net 27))
 (segment (start 97.34 144.71) (end 97.34 147.25) (width 0.25) (layer F.Cu) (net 28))
 (segment (start 98.515001 143.534999) (end 97.34 144.71) (width 0.25) (layer F.Cu) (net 28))
 (segment (start 107.244999 143.534999) (end 98.515001 143.534999) (width 0.25) (layer F.Cu) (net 28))
 (segment (start 107.4 143.69) (end 107.244999 143.534999) (width 0.25) (layer F.Cu) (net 28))
 (segment (start 107.4 144.79) (end 107.4 143.69) (width 0.25) (layer F.Cu) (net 28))
 (segment (start 94.8 144.71) (end 94.8 147.25) (width 0.25) (layer F.Cu) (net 29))
 (segment (start 111.304999 145.965001) (end 112.48 144.79) (width 0.25) (layer F.Cu) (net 29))
 (segment (start 106.509997 145.965001) (end 111.304999 145.965001) (width 0.25) (layer F.Cu) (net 29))
 (segment (start 104.049997 148.425001) (end 106.509997 145.965001) (width 0.25) (layer F.Cu) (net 29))
 (segment (start 95.975001 148.425001) (end 104.049997 148.425001) (width 0.25) (layer F.Cu) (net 29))
 (segment (start 94.8 147.25) (end 95.975001 148.425001) (width 0.25) (layer F.Cu) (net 29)))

